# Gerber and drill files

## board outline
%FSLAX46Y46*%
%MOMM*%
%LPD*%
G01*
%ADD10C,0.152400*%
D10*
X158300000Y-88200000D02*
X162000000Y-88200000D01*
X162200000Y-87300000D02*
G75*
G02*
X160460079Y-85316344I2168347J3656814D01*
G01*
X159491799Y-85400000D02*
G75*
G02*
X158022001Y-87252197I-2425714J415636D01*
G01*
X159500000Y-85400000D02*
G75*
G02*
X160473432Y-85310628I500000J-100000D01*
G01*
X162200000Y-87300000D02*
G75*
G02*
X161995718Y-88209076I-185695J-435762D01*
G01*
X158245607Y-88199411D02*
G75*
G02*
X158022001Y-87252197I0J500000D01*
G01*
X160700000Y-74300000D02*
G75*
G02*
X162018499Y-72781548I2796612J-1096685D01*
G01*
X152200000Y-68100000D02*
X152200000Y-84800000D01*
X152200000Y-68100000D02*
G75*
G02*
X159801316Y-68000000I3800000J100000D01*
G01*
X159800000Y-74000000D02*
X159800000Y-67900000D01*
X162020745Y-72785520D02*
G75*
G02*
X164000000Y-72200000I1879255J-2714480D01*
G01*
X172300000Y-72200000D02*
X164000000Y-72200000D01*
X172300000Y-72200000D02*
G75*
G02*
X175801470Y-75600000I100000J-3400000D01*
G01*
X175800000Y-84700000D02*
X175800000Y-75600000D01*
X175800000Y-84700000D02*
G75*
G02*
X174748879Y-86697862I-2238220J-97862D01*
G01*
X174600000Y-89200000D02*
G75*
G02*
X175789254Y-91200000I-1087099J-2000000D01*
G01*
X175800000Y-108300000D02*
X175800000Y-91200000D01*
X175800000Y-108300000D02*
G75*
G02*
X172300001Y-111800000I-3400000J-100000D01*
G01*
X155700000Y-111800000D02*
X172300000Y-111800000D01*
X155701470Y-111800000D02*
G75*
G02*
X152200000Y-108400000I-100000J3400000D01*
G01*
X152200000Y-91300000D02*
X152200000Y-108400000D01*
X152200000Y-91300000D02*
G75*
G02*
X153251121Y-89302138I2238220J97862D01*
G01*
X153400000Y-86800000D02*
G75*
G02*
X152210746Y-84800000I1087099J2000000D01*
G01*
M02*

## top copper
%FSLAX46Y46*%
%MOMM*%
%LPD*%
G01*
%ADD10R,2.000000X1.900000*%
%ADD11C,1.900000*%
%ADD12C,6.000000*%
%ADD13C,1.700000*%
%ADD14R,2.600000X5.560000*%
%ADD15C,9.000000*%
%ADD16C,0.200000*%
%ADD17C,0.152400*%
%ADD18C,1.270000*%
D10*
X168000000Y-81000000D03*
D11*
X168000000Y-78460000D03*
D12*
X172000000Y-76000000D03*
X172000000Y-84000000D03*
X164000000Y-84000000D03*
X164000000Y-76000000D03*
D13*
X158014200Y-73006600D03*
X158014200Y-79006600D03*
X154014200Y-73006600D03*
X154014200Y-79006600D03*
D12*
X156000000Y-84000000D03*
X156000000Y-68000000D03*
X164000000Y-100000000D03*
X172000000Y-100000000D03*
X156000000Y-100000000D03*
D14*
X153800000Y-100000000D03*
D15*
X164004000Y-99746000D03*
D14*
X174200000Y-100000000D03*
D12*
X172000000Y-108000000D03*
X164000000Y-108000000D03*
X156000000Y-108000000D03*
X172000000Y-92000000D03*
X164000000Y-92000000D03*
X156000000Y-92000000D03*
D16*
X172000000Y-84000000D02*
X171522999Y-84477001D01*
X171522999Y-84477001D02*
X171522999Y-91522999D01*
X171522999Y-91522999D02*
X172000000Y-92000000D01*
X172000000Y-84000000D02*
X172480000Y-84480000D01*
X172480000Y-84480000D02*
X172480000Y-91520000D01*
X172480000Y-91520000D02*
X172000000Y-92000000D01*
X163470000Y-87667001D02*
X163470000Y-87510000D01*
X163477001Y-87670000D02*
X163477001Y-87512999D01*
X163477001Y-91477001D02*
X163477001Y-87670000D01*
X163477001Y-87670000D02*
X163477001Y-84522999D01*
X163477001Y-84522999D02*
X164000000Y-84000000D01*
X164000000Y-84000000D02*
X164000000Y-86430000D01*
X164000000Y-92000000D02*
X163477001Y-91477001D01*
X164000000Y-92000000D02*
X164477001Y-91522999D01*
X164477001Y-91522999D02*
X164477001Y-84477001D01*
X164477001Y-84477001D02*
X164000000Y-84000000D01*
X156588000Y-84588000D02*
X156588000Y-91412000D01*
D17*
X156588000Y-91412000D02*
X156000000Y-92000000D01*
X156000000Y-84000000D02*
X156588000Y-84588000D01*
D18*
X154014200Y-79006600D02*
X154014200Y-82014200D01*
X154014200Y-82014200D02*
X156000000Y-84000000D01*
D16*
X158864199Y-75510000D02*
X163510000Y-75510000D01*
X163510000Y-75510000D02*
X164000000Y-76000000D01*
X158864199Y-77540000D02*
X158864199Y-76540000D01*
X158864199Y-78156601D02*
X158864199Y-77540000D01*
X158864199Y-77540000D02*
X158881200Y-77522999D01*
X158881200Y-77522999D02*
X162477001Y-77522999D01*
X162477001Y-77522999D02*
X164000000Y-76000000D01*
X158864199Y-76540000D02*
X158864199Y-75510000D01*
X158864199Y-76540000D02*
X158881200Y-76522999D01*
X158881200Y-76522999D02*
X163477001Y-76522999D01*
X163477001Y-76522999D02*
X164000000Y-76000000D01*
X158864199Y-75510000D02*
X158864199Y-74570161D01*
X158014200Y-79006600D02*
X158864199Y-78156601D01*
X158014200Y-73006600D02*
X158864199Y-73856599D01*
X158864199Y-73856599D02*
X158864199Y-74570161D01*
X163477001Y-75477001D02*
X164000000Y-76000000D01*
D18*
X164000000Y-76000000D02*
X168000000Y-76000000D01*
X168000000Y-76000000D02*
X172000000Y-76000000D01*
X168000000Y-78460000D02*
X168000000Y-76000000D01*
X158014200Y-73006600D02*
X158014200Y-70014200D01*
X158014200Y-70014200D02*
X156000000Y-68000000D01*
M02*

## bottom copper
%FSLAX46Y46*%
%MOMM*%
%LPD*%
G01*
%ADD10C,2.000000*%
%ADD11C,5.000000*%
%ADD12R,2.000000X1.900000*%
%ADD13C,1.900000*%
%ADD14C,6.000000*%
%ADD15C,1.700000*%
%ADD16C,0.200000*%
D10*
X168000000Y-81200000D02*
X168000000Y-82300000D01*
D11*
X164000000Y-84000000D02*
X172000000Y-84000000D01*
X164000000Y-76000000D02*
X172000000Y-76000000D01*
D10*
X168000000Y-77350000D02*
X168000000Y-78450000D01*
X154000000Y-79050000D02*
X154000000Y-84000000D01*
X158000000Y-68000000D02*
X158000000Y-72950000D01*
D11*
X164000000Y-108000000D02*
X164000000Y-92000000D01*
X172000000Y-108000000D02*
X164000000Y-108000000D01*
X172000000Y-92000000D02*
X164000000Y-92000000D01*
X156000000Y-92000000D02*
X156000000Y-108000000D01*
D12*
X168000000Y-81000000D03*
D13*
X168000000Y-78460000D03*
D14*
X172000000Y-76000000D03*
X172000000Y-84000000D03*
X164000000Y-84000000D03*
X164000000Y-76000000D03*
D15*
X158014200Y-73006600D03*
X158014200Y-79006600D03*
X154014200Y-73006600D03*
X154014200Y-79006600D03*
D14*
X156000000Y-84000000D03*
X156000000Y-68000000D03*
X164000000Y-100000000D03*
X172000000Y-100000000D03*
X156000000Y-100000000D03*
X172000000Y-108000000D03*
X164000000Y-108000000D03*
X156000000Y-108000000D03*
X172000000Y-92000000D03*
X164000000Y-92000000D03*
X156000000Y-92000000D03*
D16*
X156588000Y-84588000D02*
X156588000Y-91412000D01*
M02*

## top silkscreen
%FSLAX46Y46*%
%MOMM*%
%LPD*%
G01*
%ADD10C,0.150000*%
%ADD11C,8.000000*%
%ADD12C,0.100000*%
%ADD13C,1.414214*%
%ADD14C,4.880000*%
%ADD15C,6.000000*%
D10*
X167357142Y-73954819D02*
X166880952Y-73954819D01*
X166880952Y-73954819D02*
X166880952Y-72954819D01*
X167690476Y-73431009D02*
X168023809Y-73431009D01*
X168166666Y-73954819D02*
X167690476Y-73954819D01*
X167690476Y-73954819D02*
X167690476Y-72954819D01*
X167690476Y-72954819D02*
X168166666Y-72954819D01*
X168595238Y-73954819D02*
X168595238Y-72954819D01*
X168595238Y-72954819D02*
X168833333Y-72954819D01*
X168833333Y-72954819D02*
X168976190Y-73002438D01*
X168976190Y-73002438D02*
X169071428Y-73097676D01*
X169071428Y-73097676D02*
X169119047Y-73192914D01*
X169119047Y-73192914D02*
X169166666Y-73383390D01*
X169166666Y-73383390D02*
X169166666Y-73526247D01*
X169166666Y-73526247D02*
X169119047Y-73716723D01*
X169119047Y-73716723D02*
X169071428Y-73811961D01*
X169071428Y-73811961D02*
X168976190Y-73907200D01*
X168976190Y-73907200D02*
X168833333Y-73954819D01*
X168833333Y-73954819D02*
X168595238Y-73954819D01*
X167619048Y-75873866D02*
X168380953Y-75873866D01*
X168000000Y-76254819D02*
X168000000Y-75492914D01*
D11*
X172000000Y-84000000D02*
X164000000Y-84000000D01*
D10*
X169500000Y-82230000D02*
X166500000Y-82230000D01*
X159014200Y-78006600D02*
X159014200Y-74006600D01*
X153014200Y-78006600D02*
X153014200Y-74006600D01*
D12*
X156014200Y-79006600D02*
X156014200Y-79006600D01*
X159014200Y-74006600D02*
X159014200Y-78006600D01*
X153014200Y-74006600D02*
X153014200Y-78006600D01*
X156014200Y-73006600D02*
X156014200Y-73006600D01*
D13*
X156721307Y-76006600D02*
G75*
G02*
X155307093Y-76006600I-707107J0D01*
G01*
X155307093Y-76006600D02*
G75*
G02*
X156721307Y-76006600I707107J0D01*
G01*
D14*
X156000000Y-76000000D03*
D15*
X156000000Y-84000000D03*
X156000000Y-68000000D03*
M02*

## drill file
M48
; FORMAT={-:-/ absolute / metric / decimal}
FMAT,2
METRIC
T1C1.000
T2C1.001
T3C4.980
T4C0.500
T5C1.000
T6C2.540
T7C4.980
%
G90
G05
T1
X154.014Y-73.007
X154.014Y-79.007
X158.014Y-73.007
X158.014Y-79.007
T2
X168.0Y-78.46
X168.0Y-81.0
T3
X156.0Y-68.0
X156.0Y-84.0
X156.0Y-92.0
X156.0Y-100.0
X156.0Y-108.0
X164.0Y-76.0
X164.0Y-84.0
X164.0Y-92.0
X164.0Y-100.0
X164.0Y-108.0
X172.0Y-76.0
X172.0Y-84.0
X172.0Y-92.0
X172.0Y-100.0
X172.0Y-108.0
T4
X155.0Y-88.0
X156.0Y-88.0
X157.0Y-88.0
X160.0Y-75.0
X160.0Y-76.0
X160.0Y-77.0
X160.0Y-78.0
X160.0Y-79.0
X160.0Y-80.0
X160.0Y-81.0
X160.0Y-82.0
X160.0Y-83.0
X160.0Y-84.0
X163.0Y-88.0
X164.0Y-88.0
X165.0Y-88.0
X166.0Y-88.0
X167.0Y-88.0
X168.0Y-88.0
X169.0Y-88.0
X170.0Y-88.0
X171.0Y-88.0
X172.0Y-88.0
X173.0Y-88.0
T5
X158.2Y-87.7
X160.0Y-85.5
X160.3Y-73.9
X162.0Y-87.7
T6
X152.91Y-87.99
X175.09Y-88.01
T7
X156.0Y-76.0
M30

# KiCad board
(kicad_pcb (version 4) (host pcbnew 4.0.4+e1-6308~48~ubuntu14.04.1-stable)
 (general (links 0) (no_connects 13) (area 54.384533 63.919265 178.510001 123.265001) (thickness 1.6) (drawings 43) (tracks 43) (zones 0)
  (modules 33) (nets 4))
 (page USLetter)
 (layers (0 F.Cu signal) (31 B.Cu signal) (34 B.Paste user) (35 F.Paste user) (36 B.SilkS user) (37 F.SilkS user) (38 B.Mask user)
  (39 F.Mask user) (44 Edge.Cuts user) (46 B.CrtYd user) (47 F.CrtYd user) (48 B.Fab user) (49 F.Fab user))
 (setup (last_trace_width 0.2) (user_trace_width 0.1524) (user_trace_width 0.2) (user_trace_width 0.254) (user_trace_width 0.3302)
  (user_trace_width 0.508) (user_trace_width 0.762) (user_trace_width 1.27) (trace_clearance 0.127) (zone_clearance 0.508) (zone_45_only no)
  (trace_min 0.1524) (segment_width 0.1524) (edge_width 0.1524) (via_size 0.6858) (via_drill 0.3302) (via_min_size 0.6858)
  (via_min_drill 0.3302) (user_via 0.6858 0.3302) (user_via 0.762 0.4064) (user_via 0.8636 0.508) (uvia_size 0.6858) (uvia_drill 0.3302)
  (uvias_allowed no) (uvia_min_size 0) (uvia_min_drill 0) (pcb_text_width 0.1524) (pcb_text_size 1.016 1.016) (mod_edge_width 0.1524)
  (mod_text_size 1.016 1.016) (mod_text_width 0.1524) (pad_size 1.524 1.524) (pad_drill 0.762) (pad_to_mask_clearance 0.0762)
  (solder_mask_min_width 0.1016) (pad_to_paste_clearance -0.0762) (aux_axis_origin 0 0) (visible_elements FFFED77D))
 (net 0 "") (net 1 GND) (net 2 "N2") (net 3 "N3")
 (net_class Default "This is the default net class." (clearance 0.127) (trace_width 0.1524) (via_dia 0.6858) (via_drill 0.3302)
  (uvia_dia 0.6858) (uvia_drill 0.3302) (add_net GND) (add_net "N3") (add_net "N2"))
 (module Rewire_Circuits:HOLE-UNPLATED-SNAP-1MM (layer F.Cu) (at 160 85.5 270)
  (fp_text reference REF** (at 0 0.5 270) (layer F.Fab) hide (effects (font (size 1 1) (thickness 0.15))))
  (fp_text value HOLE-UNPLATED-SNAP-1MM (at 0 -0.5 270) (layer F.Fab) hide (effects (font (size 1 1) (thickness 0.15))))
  (pad "" np_thru_hole circle (at 0 0 270) (size 1 1) (drill 1) (layers *.Cu)))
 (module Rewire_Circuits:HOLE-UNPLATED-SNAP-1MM (layer F.Cu) (at 160.3 73.9)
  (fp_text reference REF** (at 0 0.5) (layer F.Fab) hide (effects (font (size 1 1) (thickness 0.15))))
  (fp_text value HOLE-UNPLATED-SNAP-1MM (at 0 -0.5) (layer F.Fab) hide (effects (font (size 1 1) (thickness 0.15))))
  (pad "" np_thru_hole circle (at 0 0) (size 1 1) (drill 1) (layers *.Cu)))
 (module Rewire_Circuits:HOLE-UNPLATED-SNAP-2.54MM (layer F.Cu) (at 175.09 88.01 180)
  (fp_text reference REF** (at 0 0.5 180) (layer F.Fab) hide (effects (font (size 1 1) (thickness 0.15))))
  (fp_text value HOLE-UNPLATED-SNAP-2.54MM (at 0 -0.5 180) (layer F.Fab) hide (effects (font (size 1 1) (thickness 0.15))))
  (pad "" np_thru_hole circle (at 0 0 180) (size 2.54 2.54) (drill 2.54) (layers *.Cu)))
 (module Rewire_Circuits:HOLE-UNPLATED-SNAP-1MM (layer F.Cu) (at 162 87.7)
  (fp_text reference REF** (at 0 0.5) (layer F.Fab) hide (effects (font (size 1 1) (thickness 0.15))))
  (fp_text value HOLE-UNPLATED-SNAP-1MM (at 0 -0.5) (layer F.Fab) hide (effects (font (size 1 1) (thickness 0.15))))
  (pad "" np_thru_hole circle (at 0 0) (size 1 1) (drill 1) (layers *.Cu)))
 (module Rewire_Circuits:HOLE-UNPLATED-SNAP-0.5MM (layer F.Cu) (at 163 88 180)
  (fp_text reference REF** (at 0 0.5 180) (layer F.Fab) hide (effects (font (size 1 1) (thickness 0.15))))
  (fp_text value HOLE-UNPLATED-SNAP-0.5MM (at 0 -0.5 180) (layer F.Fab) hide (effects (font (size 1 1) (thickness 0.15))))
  (pad "" np_thru_hole circle (at 0 0 180) (size 0.5 0.5) (drill 0.5) (layers *.Cu)))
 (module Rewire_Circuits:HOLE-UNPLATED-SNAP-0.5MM (layer F.Cu) (at 164 88 180)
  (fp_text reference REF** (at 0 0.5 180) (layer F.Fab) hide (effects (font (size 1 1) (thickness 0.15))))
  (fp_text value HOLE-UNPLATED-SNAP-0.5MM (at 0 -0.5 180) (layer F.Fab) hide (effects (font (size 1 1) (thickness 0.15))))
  (pad "" np_thru_hole circle (at 0 0 180) (size 0.5 0.5) (drill 0.5) (layers *.Cu)))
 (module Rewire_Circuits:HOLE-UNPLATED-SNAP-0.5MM (layer F.Cu) (at 173 88 180)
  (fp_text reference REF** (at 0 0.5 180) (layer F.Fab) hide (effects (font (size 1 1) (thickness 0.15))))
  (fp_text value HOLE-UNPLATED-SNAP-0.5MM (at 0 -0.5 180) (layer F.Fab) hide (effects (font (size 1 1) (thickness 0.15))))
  (pad "" np_thru_hole circle (at 0 0 180) (size 0.5 0.5) (drill 0.5) (layers *.Cu)))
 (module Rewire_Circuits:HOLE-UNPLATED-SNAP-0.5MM (layer F.Cu) (at 172 88 180)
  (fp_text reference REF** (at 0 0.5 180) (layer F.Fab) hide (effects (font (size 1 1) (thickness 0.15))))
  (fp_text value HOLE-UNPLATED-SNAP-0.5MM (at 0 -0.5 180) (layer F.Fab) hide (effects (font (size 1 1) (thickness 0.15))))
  (pad "" np_thru_hole circle (at 0 0 180) (size 0.5 0.5) (drill 0.5) (layers *.Cu)))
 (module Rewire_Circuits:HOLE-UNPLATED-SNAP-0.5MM (layer F.Cu) (at 171 88 180)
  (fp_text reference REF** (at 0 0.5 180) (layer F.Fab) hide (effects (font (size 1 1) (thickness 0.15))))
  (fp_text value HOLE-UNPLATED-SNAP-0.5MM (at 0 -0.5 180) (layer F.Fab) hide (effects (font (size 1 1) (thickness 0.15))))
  (pad "" np_thru_hole circle (at 0 0 180) (size 0.5 0.5) (drill 0.5) (layers *.Cu)))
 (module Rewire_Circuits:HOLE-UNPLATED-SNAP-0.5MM (layer F.Cu) (at 169 88 180)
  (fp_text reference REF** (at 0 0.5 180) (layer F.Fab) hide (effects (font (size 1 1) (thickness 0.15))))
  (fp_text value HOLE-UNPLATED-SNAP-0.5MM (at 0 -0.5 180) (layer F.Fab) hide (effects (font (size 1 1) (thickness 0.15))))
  (pad "" np_thru_hole circle (at 0 0 180) (size 0.5 0.5) (drill 0.5) (layers *.Cu)))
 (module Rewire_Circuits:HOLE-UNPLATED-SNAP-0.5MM (layer F.Cu) (at 170 88 180)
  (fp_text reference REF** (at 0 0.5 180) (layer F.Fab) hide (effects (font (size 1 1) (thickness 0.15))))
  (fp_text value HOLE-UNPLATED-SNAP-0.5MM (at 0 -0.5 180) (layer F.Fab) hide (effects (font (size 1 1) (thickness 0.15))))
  (pad "" np_thru_hole circle (at 0 0 180) (size 0.5 0.5) (drill 0.5) (layers *.Cu)))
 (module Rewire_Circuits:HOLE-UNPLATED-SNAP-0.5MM (layer F.Cu) (at 168 88 180)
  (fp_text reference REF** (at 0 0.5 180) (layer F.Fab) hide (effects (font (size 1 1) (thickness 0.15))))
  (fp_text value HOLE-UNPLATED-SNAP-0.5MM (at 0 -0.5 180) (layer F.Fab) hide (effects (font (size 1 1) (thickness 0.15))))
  (pad "" np_thru_hole circle (at 0 0 180) (size 0.5 0.5) (drill 0.5) (layers *.Cu)))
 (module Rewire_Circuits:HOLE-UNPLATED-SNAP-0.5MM (layer F.Cu) (at 165 88 180)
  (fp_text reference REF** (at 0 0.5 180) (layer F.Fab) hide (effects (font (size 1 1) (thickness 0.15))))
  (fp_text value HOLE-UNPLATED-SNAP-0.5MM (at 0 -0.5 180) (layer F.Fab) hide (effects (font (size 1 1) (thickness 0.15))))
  (pad "" np_thru_hole circle (at 0 0 180) (size 0.5 0.5) (drill 0.5) (layers *.Cu)))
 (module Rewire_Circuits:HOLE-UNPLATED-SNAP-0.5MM (layer F.Cu) (at 166 88 180)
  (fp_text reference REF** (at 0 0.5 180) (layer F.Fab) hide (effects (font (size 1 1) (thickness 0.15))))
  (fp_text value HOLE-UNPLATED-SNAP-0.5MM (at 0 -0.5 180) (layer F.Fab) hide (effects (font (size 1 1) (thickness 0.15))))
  (pad "" np_thru_hole circle (at 0 0 180) (size 0.5 0.5) (drill 0.5) (layers *.Cu)))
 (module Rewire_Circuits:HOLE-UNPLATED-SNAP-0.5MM (layer F.Cu) (at 167 88 180)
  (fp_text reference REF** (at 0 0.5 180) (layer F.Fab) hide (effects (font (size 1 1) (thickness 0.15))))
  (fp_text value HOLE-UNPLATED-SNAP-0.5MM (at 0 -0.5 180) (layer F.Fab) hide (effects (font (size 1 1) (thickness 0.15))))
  (pad "" np_thru_hole circle (at 0 0 180) (size 0.5 0.5) (drill 0.5) (layers *.Cu)))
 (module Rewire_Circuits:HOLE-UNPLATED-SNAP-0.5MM (layer F.Cu) (at 160 75 90)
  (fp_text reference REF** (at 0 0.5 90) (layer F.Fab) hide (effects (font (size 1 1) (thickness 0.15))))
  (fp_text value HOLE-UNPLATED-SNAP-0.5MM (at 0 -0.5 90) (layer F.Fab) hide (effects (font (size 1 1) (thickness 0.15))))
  (pad "" np_thru_hole circle (at 0 0 90) (size 0.5 0.5) (drill 0.5) (layers *.Cu)))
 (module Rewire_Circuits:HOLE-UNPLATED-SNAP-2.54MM (layer F.Cu) (at 152.91 87.99)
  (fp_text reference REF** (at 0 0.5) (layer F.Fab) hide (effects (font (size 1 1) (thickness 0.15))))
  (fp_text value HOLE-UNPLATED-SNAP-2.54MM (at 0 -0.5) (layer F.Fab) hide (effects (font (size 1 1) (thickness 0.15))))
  (pad "" np_thru_hole circle (at 0 0) (size 2.54 2.54) (drill 2.54) (layers *.Cu)))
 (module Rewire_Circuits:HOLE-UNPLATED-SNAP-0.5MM (layer F.Cu) (at 160 84 90)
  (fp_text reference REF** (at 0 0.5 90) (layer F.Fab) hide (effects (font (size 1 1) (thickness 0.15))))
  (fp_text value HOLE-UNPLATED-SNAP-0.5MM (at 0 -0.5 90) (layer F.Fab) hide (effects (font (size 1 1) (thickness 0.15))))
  (pad "" np_thru_hole circle (at 0 0 90) (size 0.5 0.5) (drill 0.5) (layers *.Cu)))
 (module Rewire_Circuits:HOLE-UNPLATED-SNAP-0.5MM (layer F.Cu) (at 160 83 90)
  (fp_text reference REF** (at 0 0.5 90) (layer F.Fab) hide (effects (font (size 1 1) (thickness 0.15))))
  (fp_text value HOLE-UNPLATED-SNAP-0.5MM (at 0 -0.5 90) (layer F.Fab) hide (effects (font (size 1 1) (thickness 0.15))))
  (pad "" np_thru_hole circle (at 0 0 90) (size 0.5 0.5) (drill 0.5) (layers *.Cu)))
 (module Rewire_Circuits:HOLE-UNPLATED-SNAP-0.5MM (layer F.Cu) (at 160 76 90)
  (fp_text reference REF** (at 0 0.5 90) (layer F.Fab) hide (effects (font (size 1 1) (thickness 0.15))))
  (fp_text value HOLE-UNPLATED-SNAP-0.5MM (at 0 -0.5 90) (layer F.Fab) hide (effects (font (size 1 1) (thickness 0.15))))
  (pad "" np_thru_hole circle (at 0 0 90) (size 0.5 0.5) (drill 0.5) (layers *.Cu)))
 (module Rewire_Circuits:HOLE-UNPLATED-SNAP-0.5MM (layer F.Cu) (at 160 77 90)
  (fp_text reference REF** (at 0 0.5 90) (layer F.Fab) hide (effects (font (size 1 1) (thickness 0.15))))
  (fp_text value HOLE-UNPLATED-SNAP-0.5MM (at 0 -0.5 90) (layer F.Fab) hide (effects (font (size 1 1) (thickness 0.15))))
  (pad "" np_thru_hole circle (at 0 0 90) (size 0.5 0.5) (drill 0.5) (layers *.Cu)))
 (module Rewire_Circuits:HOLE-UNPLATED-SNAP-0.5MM (layer F.Cu) (at 160 78 90)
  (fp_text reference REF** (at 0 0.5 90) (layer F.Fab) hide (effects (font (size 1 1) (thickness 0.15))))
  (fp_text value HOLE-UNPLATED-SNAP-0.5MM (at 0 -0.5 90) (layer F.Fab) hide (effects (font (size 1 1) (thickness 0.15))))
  (pad "" np_thru_hole circle (at 0 0 90) (size 0.5 0.5) (drill 0.5) (layers *.Cu)))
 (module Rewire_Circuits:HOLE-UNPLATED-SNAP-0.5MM (layer F.Cu) (at 160 79 90)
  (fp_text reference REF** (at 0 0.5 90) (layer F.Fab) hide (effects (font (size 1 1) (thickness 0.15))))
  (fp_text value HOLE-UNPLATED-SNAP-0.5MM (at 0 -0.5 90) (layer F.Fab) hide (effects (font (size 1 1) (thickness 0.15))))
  (pad "" np_thru_hole circle (at 0 0 90) (size 0.5 0.5) (drill 0.5) (layers *.Cu)))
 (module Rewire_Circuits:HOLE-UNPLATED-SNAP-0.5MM (layer F.Cu) (at 160 80 90)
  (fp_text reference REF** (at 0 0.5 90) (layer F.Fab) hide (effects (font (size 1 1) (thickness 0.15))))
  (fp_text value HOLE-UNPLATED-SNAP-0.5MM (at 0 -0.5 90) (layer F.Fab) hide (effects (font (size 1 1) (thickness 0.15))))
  (pad "" np_thru_hole circle (at 0 0 90) (size 0.5 0.5) (drill 0.5) (layers *.Cu)))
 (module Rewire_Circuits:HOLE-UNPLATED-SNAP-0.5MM (layer F.Cu) (at 160 81 90)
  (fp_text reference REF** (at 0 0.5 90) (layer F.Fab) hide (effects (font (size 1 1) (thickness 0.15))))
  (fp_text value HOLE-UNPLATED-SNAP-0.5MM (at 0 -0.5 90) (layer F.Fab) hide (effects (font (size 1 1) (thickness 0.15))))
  (pad "" np_thru_hole circle (at 0 0 90) (size 0.5 0.5) (drill 0.5) (layers *.Cu)))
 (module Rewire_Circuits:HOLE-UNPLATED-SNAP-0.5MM (layer F.Cu) (at 160 82 90)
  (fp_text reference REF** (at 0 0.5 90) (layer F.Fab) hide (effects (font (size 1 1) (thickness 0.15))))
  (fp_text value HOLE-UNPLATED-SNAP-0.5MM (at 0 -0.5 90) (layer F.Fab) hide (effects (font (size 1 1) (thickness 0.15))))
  (pad "" np_thru_hole circle (at 0 0 90) (size 0.5 0.5) (drill 0.5) (layers *.Cu)))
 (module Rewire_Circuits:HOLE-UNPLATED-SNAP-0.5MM (layer F.Cu) (at 155 88)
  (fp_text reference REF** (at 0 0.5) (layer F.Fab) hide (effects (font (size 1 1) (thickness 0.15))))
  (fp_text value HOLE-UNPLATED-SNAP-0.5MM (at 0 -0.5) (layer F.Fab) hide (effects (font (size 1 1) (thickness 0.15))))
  (pad "" np_thru_hole circle (at 0 0) (size 0.5 0.5) (drill 0.5) (layers *.Cu)))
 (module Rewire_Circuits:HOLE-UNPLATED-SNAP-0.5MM (layer F.Cu) (at 157 88)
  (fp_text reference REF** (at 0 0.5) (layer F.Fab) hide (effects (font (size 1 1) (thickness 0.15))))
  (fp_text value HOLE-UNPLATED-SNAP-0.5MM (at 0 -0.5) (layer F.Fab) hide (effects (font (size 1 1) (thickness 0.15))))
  (pad "" np_thru_hole circle (at 0 0) (size 0.5 0.5) (drill 0.5) (layers *.Cu)))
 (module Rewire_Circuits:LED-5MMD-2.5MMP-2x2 (layer F.Cu) (at 168 80 180)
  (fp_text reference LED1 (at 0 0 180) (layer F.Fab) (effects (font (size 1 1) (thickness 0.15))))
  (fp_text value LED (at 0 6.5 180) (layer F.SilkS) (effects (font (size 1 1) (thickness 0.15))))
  (fp_line (start 0 -1.2) (end 0 -2.3) (layer B.Cu) (width 2))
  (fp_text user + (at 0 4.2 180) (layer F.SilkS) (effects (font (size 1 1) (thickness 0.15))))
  (fp_line (start -4 -4) (end 4 -4) (layer F.SilkS) (width 8))
  (fp_line (start -1.5 -2.23) (end 1.5 -2.23) (layer F.SilkS) (width 0.15)) (fp_line (start 4 -4) (end -4 -4) (layer B.Cu) (width 5))
  (fp_line (start 4 4) (end -4 4) (layer B.Cu) (width 5)) (fp_line (start 0 2.65) (end 0 1.55) (layer B.Cu) (width 2))
  (pad - thru_hole rect (at 0 -1 180) (size 2 1.9) (drill 1.00076) (layers *.Cu *.Mask) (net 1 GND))
  (pad + thru_hole circle (at 0 1.54 90) (size 1.9 1.9) (drill 1.00076) (layers *.Cu *.Mask) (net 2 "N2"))
  (pad + thru_hole circle (at -4 4 180) (size 6 6) (drill 4.98) (layers *.Cu *.Mask) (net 2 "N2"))
  (pad - thru_hole circle (at -4 -4 180) (size 6 6) (drill 4.98) (layers *.Cu *.Mask) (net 1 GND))
  (pad - thru_hole circle (at 4 -4 180) (size 6 6) (drill 4.98) (layers *.Cu *.Mask) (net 1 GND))
  (pad + thru_hole circle (at 4 4 180) (size 6 6) (drill 4.98) (layers *.Cu *.Mask) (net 2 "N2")))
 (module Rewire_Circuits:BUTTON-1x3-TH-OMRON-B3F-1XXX (layer F.Cu) (at 156 76 90)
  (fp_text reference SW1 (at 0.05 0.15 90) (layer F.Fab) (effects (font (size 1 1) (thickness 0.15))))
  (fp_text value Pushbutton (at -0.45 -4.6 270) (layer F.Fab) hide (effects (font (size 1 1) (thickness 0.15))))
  (fp_line (start -3.05 -2) (end -8 -2) (layer B.Cu) (width 2))
  (fp_line (start -2.0066 3.0142) (end 1.9934 3.0142) (layer F.SilkS) (width 0.15))
  (fp_line (start -2.0066 -2.9858) (end 1.9934 -2.9858) (layer F.SilkS) (width 0.15))
  (fp_line (start -3.0066 0.0142) (end -3.0066 0.0142) (layer F.SilkS) (width 0))
  (fp_line (start 1.9934 3.0142) (end -2.0066 3.0142) (layer F.SilkS) (width 0))
  (fp_line (start 1.9934 -2.9858) (end -2.0066 -2.9858) (layer F.SilkS) (width 0))
  (fp_line (start 2.9934 0.0142) (end 2.9934 0.0142) (layer F.SilkS) (width 0))
  (fp_circle (center -0.0066 0.0142) (end 0.9934 1.0142) (layer F.SilkS) (width 0))
  (fp_line (start 8 2) (end 3.05 2) (layer B.Cu) (width 2))
  (pad 2 thru_hole circle (at 2.9934 2.0142 90) (size 1.7 1.7) (drill 1) (layers *.Cu *.Mask) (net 2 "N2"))
  (pad 2 thru_hole circle (at -3.0066 2.0142 90) (size 1.7 1.7) (drill 1) (layers *.Cu *.Mask) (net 2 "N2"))
  (pad 1 thru_hole circle (at 2.9934 -1.9858 90) (size 1.7 1.7) (drill 1) (layers *.Cu *.Mask) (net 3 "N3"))
  (pad 1 thru_hole circle (at -3.0066 -1.9858 90) (size 1.7 1.7) (drill 1) (layers *.Cu *.Mask) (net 3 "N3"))
  (pad "" np_thru_hole circle (at 0 0 90) (size 4.88 4.88) (drill 4.98) (layers *.Cu *.Mask F.SilkS))
  (pad 1 thru_hole circle (at -8 0 90) (size 6 6) (drill 4.98) (layers *.Cu *.Mask F.SilkS) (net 3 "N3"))
  (pad 2 thru_hole circle (at 8 0 90) (size 6 6) (drill 4.98) (layers *.Cu *.Mask F.SilkS) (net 2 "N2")))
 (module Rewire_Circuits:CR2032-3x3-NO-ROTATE (layer F.Cu) (at 164 100 180)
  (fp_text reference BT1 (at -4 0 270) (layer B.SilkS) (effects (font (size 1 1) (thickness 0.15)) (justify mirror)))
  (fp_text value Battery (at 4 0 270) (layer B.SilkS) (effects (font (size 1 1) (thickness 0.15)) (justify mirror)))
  (fp_line (start 0 -8) (end 0 8) (layer B.Cu) (width 5)) (fp_line (start -8 -8) (end 0 -8) (layer B.Cu) (width 5))
  (fp_line (start -8 8) (end 0 8) (layer B.Cu) (width 5)) (fp_line (start 8 8) (end 8 -8) (layer B.Cu) (width 5))
  (pad GND thru_hole circle (at 0 0 180) (size 6 6) (drill 4.98) (layers *.Cu *.Mask) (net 1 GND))
  (pad + thru_hole circle (at -8 0 180) (size 6 6) (drill 4.98) (layers *.Cu *.Mask) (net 3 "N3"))
  (pad + thru_hole circle (at 8 0 180) (size 6 6) (drill 4.98) (layers *.Cu *.Mask) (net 3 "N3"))
  (pad + smd rect (at 10.2 0 180) (size 2.6 5.56) (layers F.Cu F.Paste F.Mask) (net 3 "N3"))
  (pad GND smd circle (at -0.004 0.254 180) (size 9 9) (layers F.Cu F.Paste F.Mask) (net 1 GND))
  (pad + smd rect (at -10.2 0 180) (size 2.6 5.56) (layers F.Cu F.Paste F.Mask) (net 3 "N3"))
  (pad GND thru_hole circle (at -8 -8 180) (size 6 6) (drill 4.98) (layers *.Cu *.Mask) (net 1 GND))
  (pad GND thru_hole circle (at 0 -8 180) (size 6 6) (drill 4.98) (layers *.Cu *.Mask) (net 1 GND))
  (pad + thru_hole circle (at 8 -8 180) (size 6 6) (drill 4.98) (layers *.Cu *.Mask) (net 3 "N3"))
  (pad GND thru_hole circle (at -8 8 180) (size 6 6) (drill 4.98) (layers *.Cu *.Mask) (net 1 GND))
  (pad GND thru_hole circle (at 0 8 180) (size 6 6) (drill 4.98) (layers *.Cu *.Mask) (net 1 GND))
  (pad + thru_hole circle (at 8 8 180) (size 6 6) (drill 4.98) (layers *.Cu *.Mask) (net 3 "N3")))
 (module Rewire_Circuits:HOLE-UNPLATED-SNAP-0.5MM (layer F.Cu) (at 156 88)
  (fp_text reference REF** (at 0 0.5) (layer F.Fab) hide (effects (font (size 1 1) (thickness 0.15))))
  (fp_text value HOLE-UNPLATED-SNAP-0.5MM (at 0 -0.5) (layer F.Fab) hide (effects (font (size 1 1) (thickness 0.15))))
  (pad "" np_thru_hole circle (at 0 0) (size 0.5 0.5) (drill 0.5) (layers *.Cu)))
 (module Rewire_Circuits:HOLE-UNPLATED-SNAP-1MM (layer F.Cu) (at 158.2 87.7)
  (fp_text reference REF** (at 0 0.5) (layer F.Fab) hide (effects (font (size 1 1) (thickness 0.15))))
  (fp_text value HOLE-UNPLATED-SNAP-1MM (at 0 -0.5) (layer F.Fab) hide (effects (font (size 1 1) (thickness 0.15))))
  (pad "" np_thru_hole circle (at 0 0) (size 1 1) (drill 1) (layers *.Cu)))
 (gr_line (start 158.3 88.2) (end 162 88.2) (layer Edge.Cuts) (width 0.1524))
 (gr_arc (start 164.368347 83.643186) (end 162.2 87.3) (angle 36.15760514) (layer Edge.Cuts) (width 0.1524))
 (gr_arc (start 157.066085 84.984364) (end 159.491799 85.4) (angle 57.42107103) (layer Edge.Cuts) (width 0.1524))
 (gr_arc (start 160 85.5) (end 159.5 85.4) (angle 146.8886998) (layer Edge.Cuts) (width 0.1524))
 (gr_arc (start 162.014305 87.735762) (end 162.2 87.3) (angle 159.1681201) (layer Edge.Cuts) (width 0.1524))
 (gr_arc (start 158.245607 87.699411) (end 158.245607 88.199411) (angle 153.4350001) (layer Edge.Cuts) (width 0.1524))
 (gr_arc (start 163.496612 75.396685) (end 160.7 74.3) (angle 39.11172728) (layer Edge.Cuts) (width 0.1524))
 (gr_line (start 152.2 68.1) (end 152.2 84.8) (layer Edge.Cuts) (width 0.1524))
 (gr_arc (start 156 68) (end 152.2 68.1) (angle 181.5074358) (layer Edge.Cuts) (width 0.1524))
 (gr_line (start 159.8 74) (end 159.8 67.9) (layer Edge.Cuts) (width 0.1524))
 (gr_arc (start 163.9 75.5) (end 164 72.2) (angle -36.43084824) (layer Edge.Cuts) (width 0.1524))
 (gr_line (start 172.3 72.2) (end 164 72.2) (layer Edge.Cuts) (width 0.1524))
 (gr_arc (start 172.4 75.6) (end 172.3 72.2) (angle 91.68468432) (layer Edge.Cuts) (width 0.1524))
 (gr_line (start 175.8 84.7) (end 175.8 75.6) (layer Edge.Cuts) (width 0.1524))
 (gr_arc (start 173.56178 84.797862) (end 174.748879 86.697862) (angle -60.50687109) (layer Edge.Cuts) (width 0.1524))
 (gr_arc (start 173.512901 91.2) (end 174.6 89.2) (angle 61.47373049) (layer Edge.Cuts) (width 0.1524))
 (gr_line (start 175.8 108.3) (end 175.8 91.2) (layer Edge.Cuts) (width 0.1524))
 (gr_arc (start 172.4 108.4) (end 175.8 108.3) (angle 93.36935229) (layer Edge.Cuts) (width 0.1524))
 (gr_line (start 155.7 111.8) (end 172.3 111.8) (layer Edge.Cuts) (width 0.1524))
 (gr_arc (start 155.60147 108.4) (end 155.70147 111.8) (angle 91.68468432) (layer Edge.Cuts) (width 0.1524))
 (gr_line (start 152.2 91.3) (end 152.2 108.4) (layer Edge.Cuts) (width 0.1524))
 (gr_arc (start 154.43822 91.202138) (end 153.251121 89.302138) (angle -60.50687109) (layer Edge.Cuts) (width 0.1524))
 (gr_arc (start 154.487099 84.8) (end 153.4 86.8) (angle 61.47373049) (layer Edge.Cuts) (width 0.1524))
 (segment (start 172 84) (end 171.522999 84.477001) (width 0.2) (layer F.Cu) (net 1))
 (segment (start 171.522999 84.477001) (end 171.522999 91.522999) (width 0.2) (layer F.Cu) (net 1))
 (segment (start 171.522999 91.522999) (end 172 92) (width 0.2) (layer F.Cu) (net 1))
 (segment (start 172 84) (end 172.48 84.48) (width 0.2) (layer F.Cu) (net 1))
 (segment (start 172.48 84.48) (end 172.48 91.52) (width 0.2) (layer F.Cu) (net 1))
 (segment (start 172.48 91.52) (end 172 92) (width 0.2) (layer F.Cu) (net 1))
 (segment (start 163.47 87.667001) (end 163.47 87.51) (width 0.2) (layer F.Cu) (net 1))
 (segment (start 163.477001 87.67) (end 163.477001 87.512999) (width 0.2) (layer F.Cu) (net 1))
 (segment (start 163.477001 91.477001) (end 163.477001 87.67) (width 0.2) (layer F.Cu) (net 1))
 (segment (start 163.477001 87.67) (end 163.477001 84.522999) (width 0.2) (layer F.Cu) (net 1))
 (segment (start 163.477001 84.522999) (end 164 84) (width 0.2) (layer F.Cu) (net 1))
 (segment (start 164 84) (end 164 86.43) (width 0.2) (layer F.Cu) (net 1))
 (segment (start 164 92) (end 163.477001 91.477001) (width 0.2) (layer F.Cu) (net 1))
 (segment (start 164 92) (end 164.477001 91.522999) (width 0.2) (layer F.Cu) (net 1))
 (segment (start 164.477001 91.522999) (end 164.477001 84.477001) (width 0.2) (layer F.Cu) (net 1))
 (segment (start 164.477001 84.477001) (end 164 84) (width 0.2) (layer F.Cu) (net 1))
 (segment (start 156.588 84.588) (end 156.588 91.412) (width 0.2) (layer B.Cu) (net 3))
 (segment (start 156.588 84.588) (end 156.588 91.412) (width 0.2) (layer F.Cu) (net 3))
 (segment (start 156.588 91.412) (end 156 92) (width 0.1524) (layer F.Cu) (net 3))
 (segment (start 156 84) (end 156.588 84.588) (width 0.1524) (layer F.Cu) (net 3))
 (segment (start 154.0142 79.0066) (end 154.0142 82.0142) (width 1.27) (layer F.Cu) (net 3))
 (segment (start 154.0142 82.0142) (end 156 84) (width 1.27) (layer F.Cu) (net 3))
 (segment (start 158.864199 75.51) (end 163.51 75.51) (width 0.2) (layer F.Cu) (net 2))
 (segment (start 163.51 75.51) (end 164 76) (width 0.2) (layer F.Cu) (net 2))
 (segment (start 158.864199 77.54) (end 158.864199 76.54) (width 0.2) (layer F.Cu) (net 2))
 (segment (start 158.864199 78.156601) (end 158.864199 77.54) (width 0.2) (layer F.Cu) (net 2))
 (segment (start 158.864199 77.54) (end 158.8812 77.522999) (width 0.2) (layer F.Cu) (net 2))
 (segment (start 158.8812 77.522999) (end 162.477001 77.522999) (width 0.2) (layer F.Cu) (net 2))
 (segment (start 162.477001 77.522999) (end 164 76) (width 0.2) (layer F.Cu) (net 2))
 (segment (start 158.864199 76.54) (end 158.864199 75.51) (width 0.2) (layer F.Cu) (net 2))
 (segment (start 158.864199 76.54) (end 158.8812 76.522999) (width 0.2) (layer F.Cu) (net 2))
 (segment (start 158.8812 76.522999) (end 163.477001 76.522999) (width 0.2) (layer F.Cu) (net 2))
 (segment (start 163.477001 76.522999) (end 164 76) (width 0.2) (layer F.Cu) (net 2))
 (segment (start 158.864199 75.51) (end 158.864199 74.570161) (width 0.2) (layer F.Cu) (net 2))
 (segment (start 158.0142 79.0066) (end 158.864199 78.156601) (width 0.2) (layer F.Cu) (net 2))
 (segment (start 158.0142 73.0066) (end 158.864199 73.856599) (width 0.2) (layer F.Cu) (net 2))
 (segment (start 158.864199 73.856599) (end 158.864199 74.570161) (width 0.2) (layer F.Cu) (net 2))
 (segment (start 163.477001 75.477001) (end 164 76) (width 0.2) (layer F.Cu) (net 2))
 (segment (start 164 76) (end 168 76) (width 1.27) (layer F.Cu) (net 2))
 (segment (start 168 76) (end 172 76) (width 1.27) (layer F.Cu) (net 2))
 (segment (start 168 78.46) (end 168 76) (width 1.27) (layer F.Cu) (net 2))
 (segment (start 158.0142 73.0066) (end 158.0142 70.0142) (width 1.27) (layer F.Cu) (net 2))
 (segment (start 158.0142 70.0142) (end 156 68) (width 1.27) (layer F.Cu) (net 2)))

